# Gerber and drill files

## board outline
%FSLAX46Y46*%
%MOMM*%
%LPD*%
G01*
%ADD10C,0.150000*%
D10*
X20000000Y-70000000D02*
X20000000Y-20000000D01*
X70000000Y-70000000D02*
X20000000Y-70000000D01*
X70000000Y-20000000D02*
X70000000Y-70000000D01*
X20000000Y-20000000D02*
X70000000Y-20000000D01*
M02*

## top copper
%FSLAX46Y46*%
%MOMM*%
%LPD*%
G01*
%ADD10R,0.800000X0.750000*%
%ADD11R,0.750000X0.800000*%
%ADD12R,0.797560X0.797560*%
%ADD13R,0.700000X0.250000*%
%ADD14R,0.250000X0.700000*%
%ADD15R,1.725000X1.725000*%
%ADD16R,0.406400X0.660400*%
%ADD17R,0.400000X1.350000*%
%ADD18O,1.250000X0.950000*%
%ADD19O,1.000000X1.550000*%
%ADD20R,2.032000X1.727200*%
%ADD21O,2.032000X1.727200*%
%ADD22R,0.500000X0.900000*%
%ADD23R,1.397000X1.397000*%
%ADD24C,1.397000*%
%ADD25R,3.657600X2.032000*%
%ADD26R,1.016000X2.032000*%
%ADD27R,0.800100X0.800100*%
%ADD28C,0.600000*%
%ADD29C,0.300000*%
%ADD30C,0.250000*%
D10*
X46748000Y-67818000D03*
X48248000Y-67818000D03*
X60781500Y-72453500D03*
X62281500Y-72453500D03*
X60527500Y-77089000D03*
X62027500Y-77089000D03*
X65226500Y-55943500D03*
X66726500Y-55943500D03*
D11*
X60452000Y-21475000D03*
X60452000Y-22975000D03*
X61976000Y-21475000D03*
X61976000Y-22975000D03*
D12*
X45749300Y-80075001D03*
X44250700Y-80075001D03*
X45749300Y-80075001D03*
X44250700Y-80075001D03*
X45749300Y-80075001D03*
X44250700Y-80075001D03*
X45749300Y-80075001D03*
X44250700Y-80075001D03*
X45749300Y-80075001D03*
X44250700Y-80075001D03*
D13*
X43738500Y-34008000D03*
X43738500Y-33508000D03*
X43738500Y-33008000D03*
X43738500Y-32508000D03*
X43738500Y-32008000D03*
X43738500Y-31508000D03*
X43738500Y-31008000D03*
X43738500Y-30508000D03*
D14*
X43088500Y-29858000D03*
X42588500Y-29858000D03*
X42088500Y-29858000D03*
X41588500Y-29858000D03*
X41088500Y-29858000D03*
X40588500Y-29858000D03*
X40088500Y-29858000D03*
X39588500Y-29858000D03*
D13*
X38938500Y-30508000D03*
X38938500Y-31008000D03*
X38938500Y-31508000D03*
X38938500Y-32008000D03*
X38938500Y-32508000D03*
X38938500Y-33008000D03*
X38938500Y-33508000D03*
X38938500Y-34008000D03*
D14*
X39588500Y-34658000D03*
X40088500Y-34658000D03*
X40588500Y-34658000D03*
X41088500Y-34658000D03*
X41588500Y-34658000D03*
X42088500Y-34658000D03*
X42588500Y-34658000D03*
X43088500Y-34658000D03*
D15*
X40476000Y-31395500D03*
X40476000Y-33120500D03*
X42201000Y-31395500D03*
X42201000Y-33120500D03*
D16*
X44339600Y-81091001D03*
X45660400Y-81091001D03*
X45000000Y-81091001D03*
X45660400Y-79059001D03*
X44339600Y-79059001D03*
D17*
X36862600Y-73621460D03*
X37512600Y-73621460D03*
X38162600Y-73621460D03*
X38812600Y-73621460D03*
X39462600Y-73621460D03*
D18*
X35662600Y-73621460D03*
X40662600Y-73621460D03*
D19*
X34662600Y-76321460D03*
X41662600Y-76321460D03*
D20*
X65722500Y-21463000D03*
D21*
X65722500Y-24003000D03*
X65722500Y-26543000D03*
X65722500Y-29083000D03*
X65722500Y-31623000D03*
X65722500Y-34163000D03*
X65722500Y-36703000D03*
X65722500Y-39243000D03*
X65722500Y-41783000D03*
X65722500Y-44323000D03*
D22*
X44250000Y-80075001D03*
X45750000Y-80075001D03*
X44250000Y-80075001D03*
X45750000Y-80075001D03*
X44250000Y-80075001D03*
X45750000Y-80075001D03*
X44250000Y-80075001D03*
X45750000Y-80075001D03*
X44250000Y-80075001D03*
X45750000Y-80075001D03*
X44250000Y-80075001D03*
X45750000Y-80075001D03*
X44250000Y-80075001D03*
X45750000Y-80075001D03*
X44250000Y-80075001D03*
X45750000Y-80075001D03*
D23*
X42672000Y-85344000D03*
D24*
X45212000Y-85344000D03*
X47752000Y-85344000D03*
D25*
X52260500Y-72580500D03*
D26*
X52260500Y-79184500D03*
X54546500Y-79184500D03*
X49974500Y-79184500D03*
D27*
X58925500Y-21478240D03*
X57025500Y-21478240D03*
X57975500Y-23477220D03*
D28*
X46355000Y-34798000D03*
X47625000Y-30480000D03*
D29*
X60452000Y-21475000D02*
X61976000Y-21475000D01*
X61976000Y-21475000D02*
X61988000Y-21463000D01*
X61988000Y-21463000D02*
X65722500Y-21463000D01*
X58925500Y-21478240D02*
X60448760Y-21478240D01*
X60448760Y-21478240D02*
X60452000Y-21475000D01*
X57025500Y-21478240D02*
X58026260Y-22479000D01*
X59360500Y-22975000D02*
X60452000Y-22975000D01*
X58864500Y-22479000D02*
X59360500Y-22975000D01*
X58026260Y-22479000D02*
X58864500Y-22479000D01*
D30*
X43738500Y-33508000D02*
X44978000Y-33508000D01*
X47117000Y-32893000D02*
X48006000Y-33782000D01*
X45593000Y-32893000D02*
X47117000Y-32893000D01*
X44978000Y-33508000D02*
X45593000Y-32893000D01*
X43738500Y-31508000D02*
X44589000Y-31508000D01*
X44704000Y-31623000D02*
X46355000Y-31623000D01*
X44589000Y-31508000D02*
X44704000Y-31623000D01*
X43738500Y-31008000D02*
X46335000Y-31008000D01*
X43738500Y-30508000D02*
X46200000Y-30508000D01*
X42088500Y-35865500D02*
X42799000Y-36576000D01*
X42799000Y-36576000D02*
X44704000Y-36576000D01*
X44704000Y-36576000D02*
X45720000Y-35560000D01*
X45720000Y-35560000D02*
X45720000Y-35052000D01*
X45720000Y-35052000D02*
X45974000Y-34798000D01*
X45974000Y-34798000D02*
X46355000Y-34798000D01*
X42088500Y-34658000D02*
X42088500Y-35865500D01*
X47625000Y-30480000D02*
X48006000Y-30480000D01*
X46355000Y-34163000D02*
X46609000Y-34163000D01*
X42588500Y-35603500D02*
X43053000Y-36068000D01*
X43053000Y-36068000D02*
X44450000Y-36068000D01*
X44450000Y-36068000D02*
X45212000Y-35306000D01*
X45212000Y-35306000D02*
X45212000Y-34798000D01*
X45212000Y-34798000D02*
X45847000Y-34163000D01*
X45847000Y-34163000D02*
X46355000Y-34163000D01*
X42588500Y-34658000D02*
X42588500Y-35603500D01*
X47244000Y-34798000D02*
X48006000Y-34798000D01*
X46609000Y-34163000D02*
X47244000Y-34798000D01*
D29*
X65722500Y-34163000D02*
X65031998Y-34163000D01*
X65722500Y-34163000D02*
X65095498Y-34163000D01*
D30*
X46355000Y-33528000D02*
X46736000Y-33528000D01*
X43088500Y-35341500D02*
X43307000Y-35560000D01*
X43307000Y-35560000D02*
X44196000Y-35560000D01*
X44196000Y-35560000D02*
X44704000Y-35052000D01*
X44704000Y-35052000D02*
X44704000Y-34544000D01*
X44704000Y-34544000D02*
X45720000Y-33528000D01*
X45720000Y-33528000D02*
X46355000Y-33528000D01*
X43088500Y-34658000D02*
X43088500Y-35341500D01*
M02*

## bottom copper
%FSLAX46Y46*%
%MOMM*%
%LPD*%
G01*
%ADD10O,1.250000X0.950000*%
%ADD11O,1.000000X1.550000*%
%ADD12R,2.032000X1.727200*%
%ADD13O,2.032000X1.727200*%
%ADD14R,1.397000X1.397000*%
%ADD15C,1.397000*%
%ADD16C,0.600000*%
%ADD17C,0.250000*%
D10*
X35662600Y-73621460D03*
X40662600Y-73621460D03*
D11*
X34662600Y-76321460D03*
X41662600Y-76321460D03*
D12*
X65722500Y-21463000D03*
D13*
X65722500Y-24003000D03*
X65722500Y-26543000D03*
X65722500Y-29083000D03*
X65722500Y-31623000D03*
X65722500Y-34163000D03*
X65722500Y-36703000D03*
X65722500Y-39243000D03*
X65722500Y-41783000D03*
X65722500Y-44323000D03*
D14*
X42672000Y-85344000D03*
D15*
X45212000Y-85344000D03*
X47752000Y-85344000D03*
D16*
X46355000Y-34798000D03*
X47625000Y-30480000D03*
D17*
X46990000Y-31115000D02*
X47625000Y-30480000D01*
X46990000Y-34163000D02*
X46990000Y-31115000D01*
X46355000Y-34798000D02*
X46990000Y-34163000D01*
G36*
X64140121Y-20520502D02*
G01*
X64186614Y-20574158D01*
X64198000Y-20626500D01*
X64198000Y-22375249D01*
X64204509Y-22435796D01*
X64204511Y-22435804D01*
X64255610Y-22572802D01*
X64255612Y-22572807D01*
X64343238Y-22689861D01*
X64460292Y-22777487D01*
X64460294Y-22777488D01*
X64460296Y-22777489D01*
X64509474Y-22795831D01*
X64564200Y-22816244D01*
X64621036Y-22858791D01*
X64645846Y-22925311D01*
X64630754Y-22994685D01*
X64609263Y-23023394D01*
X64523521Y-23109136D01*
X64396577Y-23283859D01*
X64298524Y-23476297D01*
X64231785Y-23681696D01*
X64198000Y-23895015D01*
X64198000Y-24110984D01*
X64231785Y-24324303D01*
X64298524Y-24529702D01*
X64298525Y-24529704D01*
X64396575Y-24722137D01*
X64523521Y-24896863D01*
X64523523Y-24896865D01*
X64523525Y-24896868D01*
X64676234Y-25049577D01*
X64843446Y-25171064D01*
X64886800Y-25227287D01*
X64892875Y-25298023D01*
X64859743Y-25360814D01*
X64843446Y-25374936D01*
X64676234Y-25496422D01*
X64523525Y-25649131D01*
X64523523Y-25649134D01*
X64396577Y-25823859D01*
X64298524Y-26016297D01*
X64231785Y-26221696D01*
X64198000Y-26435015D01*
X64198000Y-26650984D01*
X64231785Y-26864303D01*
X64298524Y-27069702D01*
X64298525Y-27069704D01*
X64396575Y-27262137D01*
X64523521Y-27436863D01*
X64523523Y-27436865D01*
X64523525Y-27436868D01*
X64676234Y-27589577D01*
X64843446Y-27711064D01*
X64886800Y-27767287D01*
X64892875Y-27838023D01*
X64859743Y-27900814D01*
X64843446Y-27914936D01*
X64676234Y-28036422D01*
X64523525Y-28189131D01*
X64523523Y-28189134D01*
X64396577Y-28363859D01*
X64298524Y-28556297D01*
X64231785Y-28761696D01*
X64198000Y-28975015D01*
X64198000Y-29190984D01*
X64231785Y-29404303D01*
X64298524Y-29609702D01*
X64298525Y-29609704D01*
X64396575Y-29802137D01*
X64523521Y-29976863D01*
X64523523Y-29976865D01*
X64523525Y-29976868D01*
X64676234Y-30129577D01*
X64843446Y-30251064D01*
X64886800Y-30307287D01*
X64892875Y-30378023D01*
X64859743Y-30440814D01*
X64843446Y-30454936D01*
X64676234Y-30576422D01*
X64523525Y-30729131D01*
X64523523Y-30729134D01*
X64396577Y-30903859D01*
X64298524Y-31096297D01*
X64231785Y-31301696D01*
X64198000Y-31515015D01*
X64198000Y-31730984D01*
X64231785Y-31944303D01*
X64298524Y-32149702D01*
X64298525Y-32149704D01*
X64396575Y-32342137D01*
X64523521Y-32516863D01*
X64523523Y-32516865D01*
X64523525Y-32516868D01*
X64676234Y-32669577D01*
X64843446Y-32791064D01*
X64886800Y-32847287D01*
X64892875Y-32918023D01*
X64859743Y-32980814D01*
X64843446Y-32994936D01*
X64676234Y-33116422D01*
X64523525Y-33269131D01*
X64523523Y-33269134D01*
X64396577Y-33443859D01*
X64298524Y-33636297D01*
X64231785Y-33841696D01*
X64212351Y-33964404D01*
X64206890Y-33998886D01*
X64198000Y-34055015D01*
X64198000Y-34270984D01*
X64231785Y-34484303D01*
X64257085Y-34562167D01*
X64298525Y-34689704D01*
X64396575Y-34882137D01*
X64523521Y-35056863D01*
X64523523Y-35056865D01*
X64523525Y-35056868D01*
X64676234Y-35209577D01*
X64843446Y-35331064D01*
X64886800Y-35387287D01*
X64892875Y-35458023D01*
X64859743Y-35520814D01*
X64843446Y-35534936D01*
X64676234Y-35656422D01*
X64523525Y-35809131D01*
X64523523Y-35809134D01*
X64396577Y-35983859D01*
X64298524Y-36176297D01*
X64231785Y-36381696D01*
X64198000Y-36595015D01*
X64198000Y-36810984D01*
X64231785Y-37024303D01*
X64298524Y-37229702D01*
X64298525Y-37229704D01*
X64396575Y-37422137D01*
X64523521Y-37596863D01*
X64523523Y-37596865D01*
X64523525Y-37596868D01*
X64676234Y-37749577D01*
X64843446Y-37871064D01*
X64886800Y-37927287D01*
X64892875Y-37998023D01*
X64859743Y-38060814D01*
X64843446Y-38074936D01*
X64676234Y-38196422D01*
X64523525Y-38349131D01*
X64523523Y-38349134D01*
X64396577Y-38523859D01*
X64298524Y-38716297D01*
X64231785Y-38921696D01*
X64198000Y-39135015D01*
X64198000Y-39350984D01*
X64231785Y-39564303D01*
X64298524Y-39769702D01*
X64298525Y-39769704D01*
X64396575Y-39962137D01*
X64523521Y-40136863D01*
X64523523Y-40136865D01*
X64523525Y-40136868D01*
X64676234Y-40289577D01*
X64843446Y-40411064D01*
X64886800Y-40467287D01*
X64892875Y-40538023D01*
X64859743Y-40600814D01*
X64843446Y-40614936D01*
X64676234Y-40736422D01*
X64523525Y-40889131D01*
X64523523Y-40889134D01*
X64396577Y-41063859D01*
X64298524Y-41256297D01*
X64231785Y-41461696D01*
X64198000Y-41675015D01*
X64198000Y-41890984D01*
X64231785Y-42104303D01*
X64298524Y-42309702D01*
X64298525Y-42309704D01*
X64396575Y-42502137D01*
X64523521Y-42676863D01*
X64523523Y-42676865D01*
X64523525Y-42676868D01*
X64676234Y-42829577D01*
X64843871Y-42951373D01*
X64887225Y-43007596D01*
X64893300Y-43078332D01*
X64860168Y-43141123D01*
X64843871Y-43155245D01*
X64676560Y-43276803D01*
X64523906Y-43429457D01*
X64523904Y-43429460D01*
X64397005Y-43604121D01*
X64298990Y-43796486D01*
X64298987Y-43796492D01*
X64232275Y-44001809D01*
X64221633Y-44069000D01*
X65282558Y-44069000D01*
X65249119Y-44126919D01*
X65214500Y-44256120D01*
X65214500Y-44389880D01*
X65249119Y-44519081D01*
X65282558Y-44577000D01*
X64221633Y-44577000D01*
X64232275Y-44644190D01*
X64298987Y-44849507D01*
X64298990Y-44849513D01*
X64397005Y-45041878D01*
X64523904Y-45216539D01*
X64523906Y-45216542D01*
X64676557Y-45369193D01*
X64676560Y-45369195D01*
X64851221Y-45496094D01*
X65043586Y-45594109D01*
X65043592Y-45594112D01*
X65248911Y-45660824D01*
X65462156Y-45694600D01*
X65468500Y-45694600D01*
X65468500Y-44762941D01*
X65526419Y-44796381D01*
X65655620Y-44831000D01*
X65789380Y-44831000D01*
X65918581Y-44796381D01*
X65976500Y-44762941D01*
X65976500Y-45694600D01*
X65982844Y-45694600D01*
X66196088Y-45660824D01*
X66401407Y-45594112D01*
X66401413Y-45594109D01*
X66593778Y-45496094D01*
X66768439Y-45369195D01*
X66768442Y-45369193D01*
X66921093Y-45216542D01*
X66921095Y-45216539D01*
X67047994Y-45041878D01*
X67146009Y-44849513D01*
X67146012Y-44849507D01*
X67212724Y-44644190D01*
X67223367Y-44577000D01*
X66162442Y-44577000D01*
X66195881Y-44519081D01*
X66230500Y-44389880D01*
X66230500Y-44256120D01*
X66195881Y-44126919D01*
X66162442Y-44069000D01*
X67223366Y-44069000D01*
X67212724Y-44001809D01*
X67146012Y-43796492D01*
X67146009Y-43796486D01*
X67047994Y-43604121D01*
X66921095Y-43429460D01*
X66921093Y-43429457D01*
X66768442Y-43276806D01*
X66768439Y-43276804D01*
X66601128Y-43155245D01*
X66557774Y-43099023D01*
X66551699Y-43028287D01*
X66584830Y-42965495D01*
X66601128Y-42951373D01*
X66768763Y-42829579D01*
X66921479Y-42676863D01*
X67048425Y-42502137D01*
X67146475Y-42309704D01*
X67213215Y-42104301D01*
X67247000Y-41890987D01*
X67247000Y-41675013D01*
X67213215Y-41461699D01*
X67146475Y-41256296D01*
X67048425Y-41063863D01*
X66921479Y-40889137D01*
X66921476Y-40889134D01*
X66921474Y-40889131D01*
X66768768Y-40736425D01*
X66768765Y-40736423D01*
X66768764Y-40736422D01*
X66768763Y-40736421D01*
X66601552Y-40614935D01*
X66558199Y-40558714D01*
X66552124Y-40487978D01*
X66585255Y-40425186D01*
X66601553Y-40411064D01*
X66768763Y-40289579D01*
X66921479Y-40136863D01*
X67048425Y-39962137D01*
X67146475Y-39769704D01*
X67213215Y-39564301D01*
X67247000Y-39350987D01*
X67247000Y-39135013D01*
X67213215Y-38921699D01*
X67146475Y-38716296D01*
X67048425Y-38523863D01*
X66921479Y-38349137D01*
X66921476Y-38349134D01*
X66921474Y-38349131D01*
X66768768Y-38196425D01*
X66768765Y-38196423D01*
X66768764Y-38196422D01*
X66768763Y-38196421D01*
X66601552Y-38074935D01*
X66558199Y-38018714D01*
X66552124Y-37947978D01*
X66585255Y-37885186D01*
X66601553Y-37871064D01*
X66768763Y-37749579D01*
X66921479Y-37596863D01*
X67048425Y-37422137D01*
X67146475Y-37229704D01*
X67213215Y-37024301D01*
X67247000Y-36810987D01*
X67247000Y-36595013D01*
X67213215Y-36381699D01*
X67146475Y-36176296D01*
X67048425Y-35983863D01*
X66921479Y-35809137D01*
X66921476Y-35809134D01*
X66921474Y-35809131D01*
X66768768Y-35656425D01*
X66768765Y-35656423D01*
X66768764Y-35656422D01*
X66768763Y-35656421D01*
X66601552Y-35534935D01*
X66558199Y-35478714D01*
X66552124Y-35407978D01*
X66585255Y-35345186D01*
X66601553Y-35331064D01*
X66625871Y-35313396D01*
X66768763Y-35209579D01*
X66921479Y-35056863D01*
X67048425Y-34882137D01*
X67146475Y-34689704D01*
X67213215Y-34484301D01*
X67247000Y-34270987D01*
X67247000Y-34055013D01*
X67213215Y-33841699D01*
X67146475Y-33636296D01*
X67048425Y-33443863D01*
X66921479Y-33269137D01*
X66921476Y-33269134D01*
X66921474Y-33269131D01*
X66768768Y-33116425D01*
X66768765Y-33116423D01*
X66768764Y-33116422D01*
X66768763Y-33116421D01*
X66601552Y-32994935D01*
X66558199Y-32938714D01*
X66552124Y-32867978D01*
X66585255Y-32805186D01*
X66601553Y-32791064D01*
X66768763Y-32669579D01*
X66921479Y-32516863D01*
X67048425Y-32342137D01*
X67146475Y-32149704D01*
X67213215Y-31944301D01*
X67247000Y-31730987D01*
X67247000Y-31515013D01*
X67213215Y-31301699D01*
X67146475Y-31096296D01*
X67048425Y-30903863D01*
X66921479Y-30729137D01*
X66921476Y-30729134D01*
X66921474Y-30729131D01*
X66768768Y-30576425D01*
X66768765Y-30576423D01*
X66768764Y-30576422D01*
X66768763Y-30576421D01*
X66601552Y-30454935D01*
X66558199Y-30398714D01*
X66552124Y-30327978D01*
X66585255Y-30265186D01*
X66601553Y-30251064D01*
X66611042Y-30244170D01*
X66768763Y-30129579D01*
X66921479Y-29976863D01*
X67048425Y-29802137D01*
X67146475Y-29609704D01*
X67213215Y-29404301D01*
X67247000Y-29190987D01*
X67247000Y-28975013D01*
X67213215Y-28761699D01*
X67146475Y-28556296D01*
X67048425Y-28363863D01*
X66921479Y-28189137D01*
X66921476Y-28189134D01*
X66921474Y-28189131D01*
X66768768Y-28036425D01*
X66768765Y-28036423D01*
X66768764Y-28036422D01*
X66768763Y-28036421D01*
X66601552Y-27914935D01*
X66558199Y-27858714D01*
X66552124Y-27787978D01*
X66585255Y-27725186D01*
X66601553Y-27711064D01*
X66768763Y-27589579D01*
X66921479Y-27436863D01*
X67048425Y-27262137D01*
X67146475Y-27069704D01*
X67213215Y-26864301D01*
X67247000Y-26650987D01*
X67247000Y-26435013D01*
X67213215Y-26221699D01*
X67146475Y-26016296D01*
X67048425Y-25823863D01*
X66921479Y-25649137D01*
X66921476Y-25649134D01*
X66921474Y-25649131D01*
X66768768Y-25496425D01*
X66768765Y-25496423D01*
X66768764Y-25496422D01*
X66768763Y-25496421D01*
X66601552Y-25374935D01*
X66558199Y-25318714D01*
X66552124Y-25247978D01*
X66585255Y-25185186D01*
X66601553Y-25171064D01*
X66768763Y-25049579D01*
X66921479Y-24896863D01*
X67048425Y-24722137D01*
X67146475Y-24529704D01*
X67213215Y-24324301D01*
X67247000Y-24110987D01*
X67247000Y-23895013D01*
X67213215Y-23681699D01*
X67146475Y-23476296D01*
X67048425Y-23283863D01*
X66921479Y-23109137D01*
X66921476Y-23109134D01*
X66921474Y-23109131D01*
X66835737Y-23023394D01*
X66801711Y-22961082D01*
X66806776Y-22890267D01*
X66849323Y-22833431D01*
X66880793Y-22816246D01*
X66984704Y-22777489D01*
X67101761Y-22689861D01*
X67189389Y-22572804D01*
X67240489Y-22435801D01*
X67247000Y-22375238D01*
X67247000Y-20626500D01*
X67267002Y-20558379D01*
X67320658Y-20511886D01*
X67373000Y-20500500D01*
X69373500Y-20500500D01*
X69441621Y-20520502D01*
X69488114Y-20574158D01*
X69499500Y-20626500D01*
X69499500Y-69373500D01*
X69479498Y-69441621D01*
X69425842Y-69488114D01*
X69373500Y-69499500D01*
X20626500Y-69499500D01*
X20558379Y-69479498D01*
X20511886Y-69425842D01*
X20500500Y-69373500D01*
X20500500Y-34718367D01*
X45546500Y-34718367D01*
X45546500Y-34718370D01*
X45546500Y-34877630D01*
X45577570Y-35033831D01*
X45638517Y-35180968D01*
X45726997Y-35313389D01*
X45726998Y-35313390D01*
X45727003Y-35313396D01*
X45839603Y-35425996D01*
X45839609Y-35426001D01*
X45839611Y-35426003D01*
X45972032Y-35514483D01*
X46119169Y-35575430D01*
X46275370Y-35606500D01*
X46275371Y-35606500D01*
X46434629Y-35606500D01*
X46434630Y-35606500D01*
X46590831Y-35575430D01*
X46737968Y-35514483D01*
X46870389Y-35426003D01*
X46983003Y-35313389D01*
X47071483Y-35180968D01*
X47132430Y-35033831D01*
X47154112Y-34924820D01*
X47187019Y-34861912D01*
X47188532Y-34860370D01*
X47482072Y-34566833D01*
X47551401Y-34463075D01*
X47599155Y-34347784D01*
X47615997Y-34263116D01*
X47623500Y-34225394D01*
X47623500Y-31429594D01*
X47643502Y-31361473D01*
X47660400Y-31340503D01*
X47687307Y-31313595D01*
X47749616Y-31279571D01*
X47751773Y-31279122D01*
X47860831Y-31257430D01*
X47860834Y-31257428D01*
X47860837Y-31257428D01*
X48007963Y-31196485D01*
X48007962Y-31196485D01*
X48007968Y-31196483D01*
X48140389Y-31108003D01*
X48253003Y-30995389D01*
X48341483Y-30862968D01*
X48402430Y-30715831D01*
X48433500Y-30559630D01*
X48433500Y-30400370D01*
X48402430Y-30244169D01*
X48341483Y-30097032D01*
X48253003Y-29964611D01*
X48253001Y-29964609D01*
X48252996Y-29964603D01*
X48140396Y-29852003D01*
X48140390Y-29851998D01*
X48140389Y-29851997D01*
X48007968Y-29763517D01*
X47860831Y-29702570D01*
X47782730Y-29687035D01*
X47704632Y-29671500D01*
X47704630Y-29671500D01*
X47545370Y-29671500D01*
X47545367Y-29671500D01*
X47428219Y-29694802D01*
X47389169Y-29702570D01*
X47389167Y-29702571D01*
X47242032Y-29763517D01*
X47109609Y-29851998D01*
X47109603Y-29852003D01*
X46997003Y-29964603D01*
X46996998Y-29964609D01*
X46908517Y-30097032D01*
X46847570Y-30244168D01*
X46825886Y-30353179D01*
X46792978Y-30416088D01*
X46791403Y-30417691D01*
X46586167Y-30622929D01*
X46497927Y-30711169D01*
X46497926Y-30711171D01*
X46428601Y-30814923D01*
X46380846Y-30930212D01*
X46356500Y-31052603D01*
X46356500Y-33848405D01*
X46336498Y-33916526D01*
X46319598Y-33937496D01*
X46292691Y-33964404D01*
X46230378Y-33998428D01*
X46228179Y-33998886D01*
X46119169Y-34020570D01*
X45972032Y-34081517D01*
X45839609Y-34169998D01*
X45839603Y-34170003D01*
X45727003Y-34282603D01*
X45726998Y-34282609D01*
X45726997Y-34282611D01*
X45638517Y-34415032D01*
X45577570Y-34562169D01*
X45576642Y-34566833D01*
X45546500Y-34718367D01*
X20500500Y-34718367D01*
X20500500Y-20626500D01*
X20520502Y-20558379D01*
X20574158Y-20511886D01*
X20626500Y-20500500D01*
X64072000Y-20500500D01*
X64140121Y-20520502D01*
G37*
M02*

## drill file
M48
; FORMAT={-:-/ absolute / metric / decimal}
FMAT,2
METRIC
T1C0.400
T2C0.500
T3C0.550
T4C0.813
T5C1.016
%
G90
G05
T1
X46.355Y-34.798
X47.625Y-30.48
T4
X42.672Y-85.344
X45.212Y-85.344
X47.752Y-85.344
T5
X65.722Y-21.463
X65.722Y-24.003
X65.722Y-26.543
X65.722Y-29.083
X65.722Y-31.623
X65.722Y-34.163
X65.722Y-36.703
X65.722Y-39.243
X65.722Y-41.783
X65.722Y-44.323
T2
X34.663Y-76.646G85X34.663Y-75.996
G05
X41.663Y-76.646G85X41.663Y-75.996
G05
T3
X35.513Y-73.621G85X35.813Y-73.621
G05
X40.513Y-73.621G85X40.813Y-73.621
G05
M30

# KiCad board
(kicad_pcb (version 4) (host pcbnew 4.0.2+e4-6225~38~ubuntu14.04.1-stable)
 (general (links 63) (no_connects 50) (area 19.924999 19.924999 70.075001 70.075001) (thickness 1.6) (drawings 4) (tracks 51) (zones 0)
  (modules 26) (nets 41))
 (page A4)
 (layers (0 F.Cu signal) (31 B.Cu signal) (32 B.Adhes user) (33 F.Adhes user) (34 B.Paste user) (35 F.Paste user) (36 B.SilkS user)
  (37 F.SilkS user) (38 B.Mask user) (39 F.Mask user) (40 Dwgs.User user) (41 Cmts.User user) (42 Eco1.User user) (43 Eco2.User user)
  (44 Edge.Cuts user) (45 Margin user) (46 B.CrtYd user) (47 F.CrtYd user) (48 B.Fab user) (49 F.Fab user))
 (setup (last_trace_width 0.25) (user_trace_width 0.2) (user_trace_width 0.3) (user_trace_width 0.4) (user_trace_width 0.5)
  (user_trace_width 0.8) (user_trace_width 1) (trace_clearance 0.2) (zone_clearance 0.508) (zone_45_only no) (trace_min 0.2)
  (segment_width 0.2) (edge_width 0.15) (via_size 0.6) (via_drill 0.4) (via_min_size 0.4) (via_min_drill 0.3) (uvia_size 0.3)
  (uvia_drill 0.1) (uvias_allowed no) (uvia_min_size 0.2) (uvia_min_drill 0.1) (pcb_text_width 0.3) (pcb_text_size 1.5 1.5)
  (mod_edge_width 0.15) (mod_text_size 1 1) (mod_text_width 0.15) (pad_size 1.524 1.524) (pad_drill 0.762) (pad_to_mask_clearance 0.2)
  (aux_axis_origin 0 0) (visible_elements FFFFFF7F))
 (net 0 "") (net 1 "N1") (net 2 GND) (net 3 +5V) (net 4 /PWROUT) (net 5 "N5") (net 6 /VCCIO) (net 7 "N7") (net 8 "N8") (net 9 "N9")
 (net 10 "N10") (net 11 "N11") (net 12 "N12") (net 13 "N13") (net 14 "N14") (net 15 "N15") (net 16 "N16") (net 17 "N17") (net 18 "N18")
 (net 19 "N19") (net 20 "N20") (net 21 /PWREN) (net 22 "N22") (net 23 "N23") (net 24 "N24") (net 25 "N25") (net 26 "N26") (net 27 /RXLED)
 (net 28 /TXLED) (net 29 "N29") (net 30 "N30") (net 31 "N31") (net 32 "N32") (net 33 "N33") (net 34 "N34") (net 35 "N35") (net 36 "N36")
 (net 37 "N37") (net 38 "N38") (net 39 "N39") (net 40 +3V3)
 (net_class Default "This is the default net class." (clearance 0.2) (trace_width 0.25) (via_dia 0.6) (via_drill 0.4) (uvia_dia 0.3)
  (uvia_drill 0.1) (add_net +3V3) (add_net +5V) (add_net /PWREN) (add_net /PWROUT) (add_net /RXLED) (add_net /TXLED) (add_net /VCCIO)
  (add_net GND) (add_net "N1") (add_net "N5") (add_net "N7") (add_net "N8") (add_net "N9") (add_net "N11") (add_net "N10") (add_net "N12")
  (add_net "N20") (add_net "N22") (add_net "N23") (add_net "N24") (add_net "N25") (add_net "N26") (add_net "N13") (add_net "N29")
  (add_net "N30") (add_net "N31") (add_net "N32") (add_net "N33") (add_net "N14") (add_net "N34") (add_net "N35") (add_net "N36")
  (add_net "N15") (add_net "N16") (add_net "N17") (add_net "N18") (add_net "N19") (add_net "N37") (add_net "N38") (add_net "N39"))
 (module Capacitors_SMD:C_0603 (layer F.Cu) (at 47.498 67.818)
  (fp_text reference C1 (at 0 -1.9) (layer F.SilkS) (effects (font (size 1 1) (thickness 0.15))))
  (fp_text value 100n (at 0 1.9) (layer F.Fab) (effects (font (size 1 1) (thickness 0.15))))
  (pad 1 smd rect (at -0.75 0) (size 0.8 0.75) (layers F.Cu F.Paste F.Mask) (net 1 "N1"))
  (pad 2 smd rect (at 0.75 0) (size 0.8 0.75) (layers F.Cu F.Paste F.Mask) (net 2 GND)))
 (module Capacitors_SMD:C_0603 (layer F.Cu) (at 61.5315 72.4535)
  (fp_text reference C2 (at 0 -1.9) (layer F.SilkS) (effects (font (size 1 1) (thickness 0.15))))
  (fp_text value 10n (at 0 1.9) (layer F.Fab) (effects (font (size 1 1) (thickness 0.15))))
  (pad 1 smd rect (at -0.75 0) (size 0.8 0.75) (layers F.Cu F.Paste F.Mask) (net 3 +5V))
  (pad 2 smd rect (at 0.75 0) (size 0.8 0.75) (layers F.Cu F.Paste F.Mask) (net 2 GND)))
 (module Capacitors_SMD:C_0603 (layer F.Cu) (at 61.2775 77.089)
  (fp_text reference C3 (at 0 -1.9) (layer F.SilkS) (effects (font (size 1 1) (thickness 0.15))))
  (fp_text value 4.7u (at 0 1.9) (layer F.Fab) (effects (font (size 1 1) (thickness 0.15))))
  (pad 1 smd rect (at -0.75 0) (size 0.8 0.75) (layers F.Cu F.Paste F.Mask) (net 3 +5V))
  (pad 2 smd rect (at 0.75 0) (size 0.8 0.75) (layers F.Cu F.Paste F.Mask) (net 2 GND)))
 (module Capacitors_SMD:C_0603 (layer F.Cu) (at 65.9765 55.9435)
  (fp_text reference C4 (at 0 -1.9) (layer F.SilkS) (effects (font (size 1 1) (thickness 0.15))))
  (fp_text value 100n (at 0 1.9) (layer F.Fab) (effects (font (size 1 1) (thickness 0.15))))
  (pad 1 smd rect (at -0.75 0) (size 0.8 0.75) (layers F.Cu F.Paste F.Mask) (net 3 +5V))
  (pad 2 smd rect (at 0.75 0) (size 0.8 0.75) (layers F.Cu F.Paste F.Mask) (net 2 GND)))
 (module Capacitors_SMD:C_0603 (layer F.Cu) (at 60.452 22.225 270)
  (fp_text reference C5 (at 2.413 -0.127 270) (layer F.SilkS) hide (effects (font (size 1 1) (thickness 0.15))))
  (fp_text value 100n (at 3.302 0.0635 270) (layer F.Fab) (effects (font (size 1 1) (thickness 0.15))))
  (pad 1 smd rect (at -0.75 0 270) (size 0.8 0.75) (layers F.Cu F.Paste F.Mask) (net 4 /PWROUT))
  (pad 2 smd rect (at 0.75 0 270) (size 0.8 0.75) (layers F.Cu F.Paste F.Mask) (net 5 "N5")))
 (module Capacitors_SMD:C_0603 (layer F.Cu) (at 61.976 22.225 270)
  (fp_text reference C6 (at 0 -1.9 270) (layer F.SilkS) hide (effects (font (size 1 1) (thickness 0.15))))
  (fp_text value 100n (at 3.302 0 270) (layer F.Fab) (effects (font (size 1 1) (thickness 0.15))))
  (pad 1 smd rect (at -0.75 0 270) (size 0.8 0.75) (layers F.Cu F.Paste F.Mask) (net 4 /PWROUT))
  (pad 2 smd rect (at 0.75 0 270) (size 0.8 0.75) (layers F.Cu F.Paste F.Mask) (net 2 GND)))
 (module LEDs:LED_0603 (layer F.Cu) (at 45 80.075001)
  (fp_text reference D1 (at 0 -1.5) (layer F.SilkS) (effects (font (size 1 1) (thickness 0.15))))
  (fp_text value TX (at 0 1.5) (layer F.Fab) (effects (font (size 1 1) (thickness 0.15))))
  (pad 2 smd rect (at 0.7493 0 180) (size 0.79756 0.79756) (layers F.Cu F.Paste F.Mask) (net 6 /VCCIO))
  (pad 1 smd rect (at -0.7493 0 180) (size 0.79756 0.79756) (layers F.Cu F.Paste F.Mask) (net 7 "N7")))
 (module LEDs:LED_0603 (layer F.Cu) (at 45 80.075001)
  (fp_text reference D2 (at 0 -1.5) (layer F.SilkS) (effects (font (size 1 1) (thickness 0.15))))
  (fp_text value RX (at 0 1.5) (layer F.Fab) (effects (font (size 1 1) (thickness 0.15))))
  (pad 2 smd rect (at 0.7493 0 180) (size 0.79756 0.79756) (layers F.Cu F.Paste F.Mask) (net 6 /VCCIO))
  (pad 1 smd rect (at -0.7493 0 180) (size 0.79756 0.79756) (layers F.Cu F.Paste F.Mask) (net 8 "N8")))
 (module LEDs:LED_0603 (layer F.Cu) (at 45 80.075001)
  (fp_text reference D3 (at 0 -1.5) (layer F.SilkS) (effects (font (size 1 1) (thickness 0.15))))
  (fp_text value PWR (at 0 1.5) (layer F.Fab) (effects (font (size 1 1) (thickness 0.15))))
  (pad 2 smd rect (at 0.7493 0 180) (size 0.79756 0.79756) (layers F.Cu F.Paste F.Mask) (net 3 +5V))
  (pad 1 smd rect (at -0.7493 0 180) (size 0.79756 0.79756) (layers F.Cu F.Paste F.Mask) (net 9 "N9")))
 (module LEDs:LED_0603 (layer F.Cu) (at 45 80.075001)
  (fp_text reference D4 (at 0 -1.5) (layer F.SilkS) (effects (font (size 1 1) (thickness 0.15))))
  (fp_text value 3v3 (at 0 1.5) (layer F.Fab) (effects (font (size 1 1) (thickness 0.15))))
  (pad 2 smd rect (at 0.7493 0 180) (size 0.79756 0.79756) (layers F.Cu F.Paste F.Mask) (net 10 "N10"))
  (pad 1 smd rect (at -0.7493 0 180) (size 0.79756 0.79756) (layers F.Cu F.Paste F.Mask) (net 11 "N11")))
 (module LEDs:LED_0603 (layer F.Cu) (at 45 80.075001)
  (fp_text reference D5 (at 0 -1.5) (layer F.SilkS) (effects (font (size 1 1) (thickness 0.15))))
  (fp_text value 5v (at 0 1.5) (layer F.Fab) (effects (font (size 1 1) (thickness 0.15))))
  (pad 2 smd rect (at 0.7493 0 180) (size 0.79756 0.79756) (layers F.Cu F.Paste F.Mask) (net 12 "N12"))
  (pad 1 smd rect (at -0.7493 0 180) (size 0.79756 0.79756) (layers F.Cu F.Paste F.Mask) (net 2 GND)))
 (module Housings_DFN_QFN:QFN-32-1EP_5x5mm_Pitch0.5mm (layer F.Cu) (at 41.3385 32.258 180)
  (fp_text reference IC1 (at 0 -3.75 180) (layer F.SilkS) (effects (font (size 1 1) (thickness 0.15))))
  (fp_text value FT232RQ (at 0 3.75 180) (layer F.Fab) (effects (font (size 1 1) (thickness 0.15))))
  (pad 1 smd rect (at -2.4 -1.75 180) (size 0.7 0.25) (layers F.Cu F.Paste F.Mask) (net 6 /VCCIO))
  (pad 2 smd rect (at -2.4 -1.25 180) (size 0.7 0.25) (layers F.Cu F.Paste F.Mask) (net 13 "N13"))
  (pad 3 smd rect (at -2.4 -0.75 180) (size 0.7 0.25) (layers F.Cu F.Paste F.Mask) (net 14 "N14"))
  (pad 4 smd rect (at -2.4 -0.25 180) (size 0.7 0.25) (layers F.Cu F.Paste F.Mask) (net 2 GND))
  (pad 5 smd rect (at -2.4 0.25 180) (size 0.7 0.25) (layers F.Cu F.Paste F.Mask) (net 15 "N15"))
  (pad 6 smd rect (at -2.4 0.75 180) (size 0.7 0.25) (layers F.Cu F.Paste F.Mask) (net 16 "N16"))
  (pad 7 smd rect (at -2.4 1.25 180) (size 0.7 0.25) (layers F.Cu F.Paste F.Mask) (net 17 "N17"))
  (pad 8 smd rect (at -2.4 1.75 180) (size 0.7 0.25) (layers F.Cu F.Paste F.Mask) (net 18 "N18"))
  (pad 9 smd rect (at -1.75 2.4 270) (size 0.7 0.25) (layers F.Cu F.Paste F.Mask) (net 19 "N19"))
  (pad 10 smd rect (at -1.25 2.4 270) (size 0.7 0.25) (layers F.Cu F.Paste F.Mask) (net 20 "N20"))
  (pad 11 smd rect (at -0.75 2.4 270) (size 0.7 0.25) (layers F.Cu F.Paste F.Mask) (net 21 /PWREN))
  (pad 12 smd rect (at -0.25 2.4 270) (size 0.7 0.25) (layers F.Cu F.Paste F.Mask) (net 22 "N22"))
  (pad 13 smd rect (at 0.25 2.4 270) (size 0.7 0.25) (layers F.Cu F.Paste F.Mask) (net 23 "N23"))
  (pad 14 smd rect (at 0.75 2.4 270) (size 0.7 0.25) (layers F.Cu F.Paste F.Mask) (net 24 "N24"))
  (pad 15 smd rect (at 1.25 2.4 270) (size 0.7 0.25) (layers F.Cu F.Paste F.Mask) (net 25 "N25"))
  (pad 16 smd rect (at 1.75 2.4 270) (size 0.7 0.25) (layers F.Cu F.Paste F.Mask) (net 1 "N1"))
  (pad 17 smd rect (at 2.4 1.75 180) (size 0.7 0.25) (layers F.Cu F.Paste F.Mask) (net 2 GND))
  (pad 18 smd rect (at 2.4 1.25 180) (size 0.7 0.25) (layers F.Cu F.Paste F.Mask) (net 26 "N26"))
  (pad 19 smd rect (at 2.4 0.75 180) (size 0.7 0.25) (layers F.Cu F.Paste F.Mask) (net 3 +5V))
  (pad 20 smd rect (at 2.4 0.25 180) (size 0.7 0.25) (layers F.Cu F.Paste F.Mask) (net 2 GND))
  (pad 21 smd rect (at 2.4 -0.25 180) (size 0.7 0.25) (layers F.Cu F.Paste F.Mask) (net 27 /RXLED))
  (pad 22 smd rect (at 2.4 -0.75 180) (size 0.7 0.25) (layers F.Cu F.Paste F.Mask) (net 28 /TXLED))
  (pad 23 smd rect (at 2.4 -1.25 180) (size 0.7 0.25) (layers F.Cu F.Paste F.Mask) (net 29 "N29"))
  (pad 24 smd rect (at 2.4 -1.75 180) (size 0.7 0.25) (layers F.Cu F.Paste F.Mask) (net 2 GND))
  (pad 25 smd rect (at 1.75 -2.4 270) (size 0.7 0.25) (layers F.Cu F.Paste F.Mask) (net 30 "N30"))
  (pad 26 smd rect (at 1.25 -2.4 270) (size 0.7 0.25) (layers F.Cu F.Paste F.Mask) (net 2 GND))
  (pad 27 smd rect (at 0.75 -2.4 270) (size 0.7 0.25) (layers F.Cu F.Paste F.Mask) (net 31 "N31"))
  (pad 28 smd rect (at 0.25 -2.4 270) (size 0.7 0.25) (layers F.Cu F.Paste F.Mask) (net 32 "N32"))
  (pad 29 smd rect (at -0.25 -2.4 270) (size 0.7 0.25) (layers F.Cu F.Paste F.Mask) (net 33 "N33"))
  (pad 30 smd rect (at -0.75 -2.4 270) (size 0.7 0.25) (layers F.Cu F.Paste F.Mask) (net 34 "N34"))
  (pad 31 smd rect (at -1.25 -2.4 270) (size 0.7 0.25) (layers F.Cu F.Paste F.Mask) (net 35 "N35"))
  (pad 32 smd rect (at -1.75 -2.4 270) (size 0.7 0.25) (layers F.Cu F.Paste F.Mask) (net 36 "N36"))
  (pad 33 smd rect (at 0.8625 0.8625 180) (size 1.725 1.725) (layers F.Cu F.Paste F.Mask) (solder_paste_margin_ratio -0.2))
  (pad 33 smd rect (at 0.8625 -0.8625 180) (size 1.725 1.725) (layers F.Cu F.Paste F.Mask) (solder_paste_margin_ratio -0.2))
  (pad 33 smd rect (at -0.8625 0.8625 180) (size 1.725 1.725) (layers F.Cu F.Paste F.Mask) (solder_paste_margin_ratio -0.2))
  (pad 33 smd rect (at -0.8625 -0.8625 180) (size 1.725 1.725) (layers F.Cu F.Paste F.Mask) (solder_paste_margin_ratio -0.2)))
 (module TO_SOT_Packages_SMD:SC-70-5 (layer F.Cu) (at 45 80.075001)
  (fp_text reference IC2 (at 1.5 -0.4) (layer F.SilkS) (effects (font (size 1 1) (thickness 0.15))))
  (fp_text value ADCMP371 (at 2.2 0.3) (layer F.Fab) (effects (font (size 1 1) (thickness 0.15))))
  (pad 1 smd rect (at -0.6604 1.016) (size 0.4064 0.6604) (layers F.Cu F.Paste F.Mask) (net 6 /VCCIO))
  (pad 3 smd rect (at 0.6604 1.016) (size 0.4064 0.6604) (layers F.Cu F.Paste F.Mask) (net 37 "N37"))
  (pad 2 smd rect (at 0 1.016) (size 0.4064 0.6604) (layers F.Cu F.Paste F.Mask) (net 2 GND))
  (pad 4 smd rect (at 0.6604 -1.016) (size 0.4064 0.6604) (layers F.Cu F.Paste F.Mask) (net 11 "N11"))
  (pad 5 smd rect (at -0.6604 -1.016) (size 0.4064 0.6604) (layers F.Cu F.Paste F.Mask) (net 3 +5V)))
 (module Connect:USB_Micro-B (layer F.Cu) (at 38.1635 75.184)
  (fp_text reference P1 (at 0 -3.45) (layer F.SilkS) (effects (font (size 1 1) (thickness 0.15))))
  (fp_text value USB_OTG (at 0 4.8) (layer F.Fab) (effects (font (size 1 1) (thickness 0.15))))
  (pad 1 smd rect (at -1.3009 -1.56254 90) (size 1.35 0.4) (layers F.Cu F.Paste F.Mask) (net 3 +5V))
  (pad 2 smd rect (at -0.6509 -1.56254 90) (size 1.35 0.4) (layers F.Cu F.Paste F.Mask) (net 25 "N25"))
  (pad 3 smd rect (at -0.0009 -1.56254 90) (size 1.35 0.4) (layers F.Cu F.Paste F.Mask) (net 24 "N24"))
  (pad 4 smd rect (at 0.6491 -1.56254 90) (size 1.35 0.4) (layers F.Cu F.Paste F.Mask) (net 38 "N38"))
  (pad 5 smd rect (at 1.2991 -1.56254 90) (size 1.35 0.4) (layers F.Cu F.Paste F.Mask) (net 2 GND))
  (pad 6 thru_hole oval (at -2.5009 -1.56254 90) (size 0.95 1.25) (drill oval 0.55 0.85) (layers *.Cu *.Mask F.SilkS) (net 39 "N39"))
  (pad 6 thru_hole oval (at 2.4991 -1.56254 90) (size 0.95 1.25) (drill oval 0.55 0.85) (layers *.Cu *.Mask F.SilkS) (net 39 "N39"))
  (pad 6 thru_hole oval (at -3.5009 1.13746 90) (size 1.55 1) (drill oval 1.15 0.5) (layers *.Cu *.Mask F.SilkS) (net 39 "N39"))
  (pad 6 thru_hole oval (at 3.4991 1.13746 90) (size 1.55 1) (drill oval 1.15 0.5) (layers *.Cu *.Mask F.SilkS) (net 39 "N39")))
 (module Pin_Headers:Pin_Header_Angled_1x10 (layer F.Cu) (at 65.7225 21.463)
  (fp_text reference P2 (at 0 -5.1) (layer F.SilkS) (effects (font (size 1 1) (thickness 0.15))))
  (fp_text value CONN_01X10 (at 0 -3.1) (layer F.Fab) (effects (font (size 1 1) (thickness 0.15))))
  (pad 1 thru_hole rect (at 0 0) (size 2.032 1.7272) (drill 1.016) (layers *.Cu *.Mask F.SilkS) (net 4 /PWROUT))
  (pad 2 thru_hole oval (at 0 2.54) (size 2.032 1.7272) (drill 1.016) (layers *.Cu *.Mask F.SilkS) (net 34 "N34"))
  (pad 3 thru_hole oval (at 0 5.08) (size 2.032 1.7272) (drill 1.016) (layers *.Cu *.Mask F.SilkS) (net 13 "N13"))
  (pad 4 thru_hole oval (at 0 7.62) (size 2.032 1.7272) (drill 1.016) (layers *.Cu *.Mask F.SilkS) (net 36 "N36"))
  (pad 5 thru_hole oval (at 0 10.16) (size 2.032 1.7272) (drill 1.016) (layers *.Cu *.Mask F.SilkS) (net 18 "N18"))
  (pad 6 thru_hole oval (at 0 12.7) (size 2.032 1.7272) (drill 1.016) (layers *.Cu *.Mask F.SilkS) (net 35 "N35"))
  (pad 7 thru_hole oval (at 0 15.24) (size 2.032 1.7272) (drill 1.016) (layers *.Cu *.Mask F.SilkS) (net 16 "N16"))
  (pad 8 thru_hole oval (at 0 17.78) (size 2.032 1.7272) (drill 1.016) (layers *.Cu *.Mask F.SilkS) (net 17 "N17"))
  (pad 9 thru_hole oval (at 0 20.32) (size 2.032 1.7272) (drill 1.016) (layers *.Cu *.Mask F.SilkS) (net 14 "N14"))
  (pad 10 thru_hole oval (at 0 22.86) (size 2.032 1.7272) (drill 1.016) (layers *.Cu *.Mask F.SilkS) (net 2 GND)))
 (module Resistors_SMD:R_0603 (layer F.Cu) (at 45 80.075001)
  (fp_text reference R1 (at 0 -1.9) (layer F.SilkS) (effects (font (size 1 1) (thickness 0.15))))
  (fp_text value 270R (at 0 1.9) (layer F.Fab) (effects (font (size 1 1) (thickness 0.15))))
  (pad 1 smd rect (at -0.75 0) (size 0.5 0.9) (layers F.Cu F.Paste F.Mask) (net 7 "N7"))
  (pad 2 smd rect (at 0.75 0) (size 0.5 0.9) (layers F.Cu F.Paste F.Mask) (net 28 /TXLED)))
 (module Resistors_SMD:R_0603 (layer F.Cu) (at 45 80.075001)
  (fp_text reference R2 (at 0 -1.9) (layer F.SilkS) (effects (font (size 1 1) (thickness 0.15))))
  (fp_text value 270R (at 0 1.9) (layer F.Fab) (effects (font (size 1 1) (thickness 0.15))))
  (pad 1 smd rect (at -0.75 0) (size 0.5 0.9) (layers F.Cu F.Paste F.Mask) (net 8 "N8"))
  (pad 2 smd rect (at 0.75 0) (size 0.5 0.9) (layers F.Cu F.Paste F.Mask) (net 27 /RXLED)))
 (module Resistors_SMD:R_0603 (layer F.Cu) (at 45 80.075001)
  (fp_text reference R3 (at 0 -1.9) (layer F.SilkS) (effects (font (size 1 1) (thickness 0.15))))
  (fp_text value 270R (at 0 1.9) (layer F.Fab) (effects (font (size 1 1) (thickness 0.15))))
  (pad 1 smd rect (at -0.75 0) (size 0.5 0.9) (layers F.Cu F.Paste F.Mask) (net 9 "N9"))
  (pad 2 smd rect (at 0.75 0) (size 0.5 0.9) (layers F.Cu F.Paste F.Mask) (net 2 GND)))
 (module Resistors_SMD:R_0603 (layer F.Cu) (at 45 80.075001)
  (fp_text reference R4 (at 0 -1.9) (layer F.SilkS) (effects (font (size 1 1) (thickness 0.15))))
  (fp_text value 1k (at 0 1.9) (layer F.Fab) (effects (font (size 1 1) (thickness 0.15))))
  (pad 1 smd rect (at -0.75 0) (size 0.5 0.9) (layers F.Cu F.Paste F.Mask) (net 5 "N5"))
  (pad 2 smd rect (at 0.75 0) (size 0.5 0.9) (layers F.Cu F.Paste F.Mask) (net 21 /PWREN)))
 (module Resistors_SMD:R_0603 (layer F.Cu) (at 45 80.075001)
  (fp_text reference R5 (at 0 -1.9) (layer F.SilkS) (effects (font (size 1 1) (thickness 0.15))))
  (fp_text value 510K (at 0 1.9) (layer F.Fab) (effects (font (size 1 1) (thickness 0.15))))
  (pad 1 smd rect (at -0.75 0) (size 0.5 0.9) (layers F.Cu F.Paste F.Mask) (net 3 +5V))
  (pad 2 smd rect (at 0.75 0) (size 0.5 0.9) (layers F.Cu F.Paste F.Mask) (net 37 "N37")))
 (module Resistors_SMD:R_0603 (layer F.Cu) (at 45 80.075001)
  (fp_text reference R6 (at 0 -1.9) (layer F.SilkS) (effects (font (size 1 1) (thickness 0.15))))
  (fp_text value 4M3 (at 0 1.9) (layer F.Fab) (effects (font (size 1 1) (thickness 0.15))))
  (pad 1 smd rect (at -0.75 0) (size 0.5 0.9) (layers F.Cu F.Paste F.Mask) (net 37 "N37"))
  (pad 2 smd rect (at 0.75 0) (size 0.5 0.9) (layers F.Cu F.Paste F.Mask) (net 2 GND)))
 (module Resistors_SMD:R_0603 (layer F.Cu) (at 45 80.075001)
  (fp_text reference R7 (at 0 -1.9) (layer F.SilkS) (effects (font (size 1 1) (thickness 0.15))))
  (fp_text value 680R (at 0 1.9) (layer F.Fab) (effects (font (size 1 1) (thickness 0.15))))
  (pad 1 smd rect (at -0.75 0) (size 0.5 0.9) (layers F.Cu F.Paste F.Mask) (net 3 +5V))
  (pad 2 smd rect (at 0.75 0) (size 0.5 0.9) (layers F.Cu F.Paste F.Mask) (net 10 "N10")))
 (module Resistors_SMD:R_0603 (layer F.Cu) (at 45 80.075001)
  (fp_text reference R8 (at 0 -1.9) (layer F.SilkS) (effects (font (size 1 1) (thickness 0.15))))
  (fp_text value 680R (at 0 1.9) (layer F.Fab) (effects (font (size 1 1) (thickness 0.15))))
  (pad 1 smd rect (at -0.75 0) (size 0.5 0.9) (layers F.Cu F.Paste F.Mask) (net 11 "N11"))
  (pad 2 smd rect (at 0.75 0) (size 0.5 0.9) (layers F.Cu F.Paste F.Mask) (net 12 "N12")))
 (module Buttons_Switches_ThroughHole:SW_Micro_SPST (layer F.Cu) (at 45.212 85.344)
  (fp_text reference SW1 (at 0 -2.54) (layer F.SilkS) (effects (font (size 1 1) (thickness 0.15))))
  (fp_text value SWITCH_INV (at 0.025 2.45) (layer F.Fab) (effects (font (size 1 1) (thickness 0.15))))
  (pad 1 thru_hole rect (at -2.54 0) (size 1.397 1.397) (drill 0.8128) (layers *.Cu *.Mask F.SilkS) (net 3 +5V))
  (pad 2 thru_hole circle (at 0 0) (size 1.397 1.397) (drill 0.8128) (layers *.Cu *.Mask F.SilkS) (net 6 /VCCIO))
  (pad 3 thru_hole circle (at 2.54 0) (size 1.397 1.397) (drill 0.8128) (layers *.Cu *.Mask F.SilkS) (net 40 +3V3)))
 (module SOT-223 (layer F.Cu) (at 52.2605 75.8825)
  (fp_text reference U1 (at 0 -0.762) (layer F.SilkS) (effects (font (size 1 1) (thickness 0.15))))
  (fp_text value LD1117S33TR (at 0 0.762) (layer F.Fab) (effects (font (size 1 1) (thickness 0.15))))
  (pad 4 smd rect (at 0 -3.302) (size 3.6576 2.032) (layers F.Cu F.Paste F.Mask))
  (pad 2 smd rect (at 0 3.302) (size 1.016 2.032) (layers F.Cu F.Paste F.Mask) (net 40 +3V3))
  (pad 3 smd rect (at 2.286 3.302) (size 1.016 2.032) (layers F.Cu F.Paste F.Mask) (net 3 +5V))
  (pad 1 smd rect (at -2.286 3.302) (size 1.016 2.032) (layers F.Cu F.Paste F.Mask) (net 2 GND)))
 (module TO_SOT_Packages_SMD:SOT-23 (layer F.Cu) (at 57.9755 22.479 180)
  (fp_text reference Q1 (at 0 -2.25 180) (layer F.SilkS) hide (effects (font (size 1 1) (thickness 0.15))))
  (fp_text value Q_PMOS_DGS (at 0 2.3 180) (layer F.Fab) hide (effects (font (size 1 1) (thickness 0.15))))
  (pad 1 smd rect (at -0.95 1.00076 180) (size 0.8001 0.8001) (layers F.Cu F.Paste F.Mask) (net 4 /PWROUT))
  (pad 2 smd rect (at 0.95 1.00076 180) (size 0.8001 0.8001) (layers F.Cu F.Paste F.Mask) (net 5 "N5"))
  (pad 3 smd rect (at 0 -0.99822 180) (size 0.8001 0.8001) (layers F.Cu F.Paste F.Mask) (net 6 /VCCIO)))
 (gr_line (start 20 70) (end 20 20) (angle 90) (layer Edge.Cuts) (width 0.15))
 (gr_line (start 70 70) (end 20 70) (angle 90) (layer Edge.Cuts) (width 0.15))
 (gr_line (start 70 20) (end 70 70) (angle 90) (layer Edge.Cuts) (width 0.15))
 (gr_line (start 20 20) (end 70 20) (angle 90) (layer Edge.Cuts) (width 0.15))
 (segment (start 60.452 21.475) (end 61.976 21.475) (width 0.3) (layer F.Cu) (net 4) (status C00000))
 (segment (start 61.976 21.475) (end 61.988 21.463) (width 0.3) (layer F.Cu) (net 4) (status C00000))
 (segment (start 61.988 21.463) (end 65.7225 21.463) (width 0.3) (layer F.Cu) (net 4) (status C00000))
 (segment (start 58.9255 21.47824) (end 60.44876 21.47824) (width 0.3) (layer F.Cu) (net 4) (status C00000))
 (segment (start 60.44876 21.47824) (end 60.452 21.475) (width 0.3) (layer F.Cu) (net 4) (status C00000))
 (segment (start 57.0255 21.47824) (end 58.02626 22.479) (width 0.3) (layer F.Cu) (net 5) (status 400000))
 (segment (start 59.3605 22.975) (end 60.452 22.975) (width 0.3) (layer F.Cu) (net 5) (status 800000))
 (segment (start 58.8645 22.479) (end 59.3605 22.975) (width 0.3) (layer F.Cu) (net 5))
 (segment (start 58.02626 22.479) (end 58.8645 22.479) (width 0.3) (layer F.Cu) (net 5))
 (segment (start 43.7385 33.508) (end 44.978 33.508) (width 0.25) (layer F.Cu) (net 13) (status 400000))
 (segment (start 47.117 32.893) (end 48.006 33.782) (width 0.25) (layer F.Cu) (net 13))
 (segment (start 45.593 32.893) (end 47.117 32.893) (width 0.25) (layer F.Cu) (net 13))
 (segment (start 44.978 33.508) (end 45.593 32.893) (width 0.25) (layer F.Cu) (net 13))
 (segment (start 43.7385 31.508) (end 44.589 31.508) (width 0.25) (layer F.Cu) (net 16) (status 400000))
 (segment (start 44.704 31.623) (end 46.355 31.623) (width 0.25) (layer F.Cu) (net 16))
 (segment (start 44.589 31.508) (end 44.704 31.623) (width 0.25) (layer F.Cu) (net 16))
 (segment (start 43.7385 31.008) (end 46.335 31.008) (width 0.25) (layer F.Cu) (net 17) (status 400000))
 (segment (start 43.7385 30.508) (end 46.2 30.508) (width 0.25) (layer F.Cu) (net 18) (status 400000))
 (via (at 46.355 34.798) (size 0.6) (drill 0.4) (layers F.Cu B.Cu) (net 34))
 (segment (start 42.0885 35.8655) (end 42.799 36.576) (width 0.25) (layer F.Cu) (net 34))
 (segment (start 42.799 36.576) (end 44.704 36.576) (width 0.25) (layer F.Cu) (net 34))
 (segment (start 44.704 36.576) (end 45.72 35.56) (width 0.25) (layer F.Cu) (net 34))
 (segment (start 45.72 35.56) (end 45.72 35.052) (width 0.25) (layer F.Cu) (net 34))
 (segment (start 45.72 35.052) (end 45.974 34.798) (width 0.25) (layer F.Cu) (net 34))
 (segment (start 45.974 34.798) (end 46.355 34.798) (width 0.25) (layer F.Cu) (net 34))
 (segment (start 42.0885 34.658) (end 42.0885 35.8655) (width 0.25) (layer F.Cu) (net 34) (status 400000))
 (segment (start 47.625 30.48) (end 48.006 30.48) (width 0.25) (layer F.Cu) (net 34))
 (via (at 47.625 30.48) (size 0.6) (drill 0.4) (layers F.Cu B.Cu) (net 34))
 (segment (start 46.99 31.115) (end 47.625 30.48) (width 0.25) (layer B.Cu) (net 34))
 (segment (start 46.99 34.163) (end 46.99 31.115) (width 0.25) (layer B.Cu) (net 34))
 (segment (start 46.355 34.798) (end 46.99 34.163) (width 0.25) (layer B.Cu) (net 34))
 (segment (start 46.355 34.163) (end 46.609 34.163) (width 0.25) (layer F.Cu) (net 35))
 (segment (start 42.5885 35.6035) (end 43.053 36.068) (width 0.25) (layer F.Cu) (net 35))
 (segment (start 43.053 36.068) (end 44.45 36.068) (width 0.25) (layer F.Cu) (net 35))
 (segment (start 44.45 36.068) (end 45.212 35.306) (width 0.25) (layer F.Cu) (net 35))
 (segment (start 45.212 35.306) (end 45.212 34.798) (width 0.25) (layer F.Cu) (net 35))
 (segment (start 45.212 34.798) (end 45.847 34.163) (width 0.25) (layer F.Cu) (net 35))
 (segment (start 45.847 34.163) (end 46.355 34.163) (width 0.25) (layer F.Cu) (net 35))
 (segment (start 42.5885 34.658) (end 42.5885 35.6035) (width 0.25) (layer F.Cu) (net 35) (status 400000))
 (segment (start 47.244 34.798) (end 48.006 34.798) (width 0.25) (layer F.Cu) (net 35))
 (segment (start 46.609 34.163) (end 47.244 34.798) (width 0.25) (layer F.Cu) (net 35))
 (segment (start 65.7225 34.163) (end 65.031998 34.163) (width 0.3) (layer F.Cu) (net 35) (status C00000))
 (segment (start 65.7225 34.163) (end 65.095498 34.163) (width 0.3) (layer F.Cu) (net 35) (status C00000))
 (segment (start 46.355 33.528) (end 46.736 33.528) (width 0.25) (layer F.Cu) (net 36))
 (segment (start 43.0885 35.3415) (end 43.307 35.56) (width 0.25) (layer F.Cu) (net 36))
 (segment (start 43.307 35.56) (end 44.196 35.56) (width 0.25) (layer F.Cu) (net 36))
 (segment (start 44.196 35.56) (end 44.704 35.052) (width 0.25) (layer F.Cu) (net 36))
 (segment (start 44.704 35.052) (end 44.704 34.544) (width 0.25) (layer F.Cu) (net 36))
 (segment (start 44.704 34.544) (end 45.72 33.528) (width 0.25) (layer F.Cu) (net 36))
 (segment (start 45.72 33.528) (end 46.355 33.528) (width 0.25) (layer F.Cu) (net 36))
 (segment (start 43.0885 34.658) (end 43.0885 35.3415) (width 0.25) (layer F.Cu) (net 36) (status 400000))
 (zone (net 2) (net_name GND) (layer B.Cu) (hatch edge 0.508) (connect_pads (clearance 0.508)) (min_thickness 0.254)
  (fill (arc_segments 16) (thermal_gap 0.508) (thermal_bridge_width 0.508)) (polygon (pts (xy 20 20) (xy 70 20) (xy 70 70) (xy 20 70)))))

